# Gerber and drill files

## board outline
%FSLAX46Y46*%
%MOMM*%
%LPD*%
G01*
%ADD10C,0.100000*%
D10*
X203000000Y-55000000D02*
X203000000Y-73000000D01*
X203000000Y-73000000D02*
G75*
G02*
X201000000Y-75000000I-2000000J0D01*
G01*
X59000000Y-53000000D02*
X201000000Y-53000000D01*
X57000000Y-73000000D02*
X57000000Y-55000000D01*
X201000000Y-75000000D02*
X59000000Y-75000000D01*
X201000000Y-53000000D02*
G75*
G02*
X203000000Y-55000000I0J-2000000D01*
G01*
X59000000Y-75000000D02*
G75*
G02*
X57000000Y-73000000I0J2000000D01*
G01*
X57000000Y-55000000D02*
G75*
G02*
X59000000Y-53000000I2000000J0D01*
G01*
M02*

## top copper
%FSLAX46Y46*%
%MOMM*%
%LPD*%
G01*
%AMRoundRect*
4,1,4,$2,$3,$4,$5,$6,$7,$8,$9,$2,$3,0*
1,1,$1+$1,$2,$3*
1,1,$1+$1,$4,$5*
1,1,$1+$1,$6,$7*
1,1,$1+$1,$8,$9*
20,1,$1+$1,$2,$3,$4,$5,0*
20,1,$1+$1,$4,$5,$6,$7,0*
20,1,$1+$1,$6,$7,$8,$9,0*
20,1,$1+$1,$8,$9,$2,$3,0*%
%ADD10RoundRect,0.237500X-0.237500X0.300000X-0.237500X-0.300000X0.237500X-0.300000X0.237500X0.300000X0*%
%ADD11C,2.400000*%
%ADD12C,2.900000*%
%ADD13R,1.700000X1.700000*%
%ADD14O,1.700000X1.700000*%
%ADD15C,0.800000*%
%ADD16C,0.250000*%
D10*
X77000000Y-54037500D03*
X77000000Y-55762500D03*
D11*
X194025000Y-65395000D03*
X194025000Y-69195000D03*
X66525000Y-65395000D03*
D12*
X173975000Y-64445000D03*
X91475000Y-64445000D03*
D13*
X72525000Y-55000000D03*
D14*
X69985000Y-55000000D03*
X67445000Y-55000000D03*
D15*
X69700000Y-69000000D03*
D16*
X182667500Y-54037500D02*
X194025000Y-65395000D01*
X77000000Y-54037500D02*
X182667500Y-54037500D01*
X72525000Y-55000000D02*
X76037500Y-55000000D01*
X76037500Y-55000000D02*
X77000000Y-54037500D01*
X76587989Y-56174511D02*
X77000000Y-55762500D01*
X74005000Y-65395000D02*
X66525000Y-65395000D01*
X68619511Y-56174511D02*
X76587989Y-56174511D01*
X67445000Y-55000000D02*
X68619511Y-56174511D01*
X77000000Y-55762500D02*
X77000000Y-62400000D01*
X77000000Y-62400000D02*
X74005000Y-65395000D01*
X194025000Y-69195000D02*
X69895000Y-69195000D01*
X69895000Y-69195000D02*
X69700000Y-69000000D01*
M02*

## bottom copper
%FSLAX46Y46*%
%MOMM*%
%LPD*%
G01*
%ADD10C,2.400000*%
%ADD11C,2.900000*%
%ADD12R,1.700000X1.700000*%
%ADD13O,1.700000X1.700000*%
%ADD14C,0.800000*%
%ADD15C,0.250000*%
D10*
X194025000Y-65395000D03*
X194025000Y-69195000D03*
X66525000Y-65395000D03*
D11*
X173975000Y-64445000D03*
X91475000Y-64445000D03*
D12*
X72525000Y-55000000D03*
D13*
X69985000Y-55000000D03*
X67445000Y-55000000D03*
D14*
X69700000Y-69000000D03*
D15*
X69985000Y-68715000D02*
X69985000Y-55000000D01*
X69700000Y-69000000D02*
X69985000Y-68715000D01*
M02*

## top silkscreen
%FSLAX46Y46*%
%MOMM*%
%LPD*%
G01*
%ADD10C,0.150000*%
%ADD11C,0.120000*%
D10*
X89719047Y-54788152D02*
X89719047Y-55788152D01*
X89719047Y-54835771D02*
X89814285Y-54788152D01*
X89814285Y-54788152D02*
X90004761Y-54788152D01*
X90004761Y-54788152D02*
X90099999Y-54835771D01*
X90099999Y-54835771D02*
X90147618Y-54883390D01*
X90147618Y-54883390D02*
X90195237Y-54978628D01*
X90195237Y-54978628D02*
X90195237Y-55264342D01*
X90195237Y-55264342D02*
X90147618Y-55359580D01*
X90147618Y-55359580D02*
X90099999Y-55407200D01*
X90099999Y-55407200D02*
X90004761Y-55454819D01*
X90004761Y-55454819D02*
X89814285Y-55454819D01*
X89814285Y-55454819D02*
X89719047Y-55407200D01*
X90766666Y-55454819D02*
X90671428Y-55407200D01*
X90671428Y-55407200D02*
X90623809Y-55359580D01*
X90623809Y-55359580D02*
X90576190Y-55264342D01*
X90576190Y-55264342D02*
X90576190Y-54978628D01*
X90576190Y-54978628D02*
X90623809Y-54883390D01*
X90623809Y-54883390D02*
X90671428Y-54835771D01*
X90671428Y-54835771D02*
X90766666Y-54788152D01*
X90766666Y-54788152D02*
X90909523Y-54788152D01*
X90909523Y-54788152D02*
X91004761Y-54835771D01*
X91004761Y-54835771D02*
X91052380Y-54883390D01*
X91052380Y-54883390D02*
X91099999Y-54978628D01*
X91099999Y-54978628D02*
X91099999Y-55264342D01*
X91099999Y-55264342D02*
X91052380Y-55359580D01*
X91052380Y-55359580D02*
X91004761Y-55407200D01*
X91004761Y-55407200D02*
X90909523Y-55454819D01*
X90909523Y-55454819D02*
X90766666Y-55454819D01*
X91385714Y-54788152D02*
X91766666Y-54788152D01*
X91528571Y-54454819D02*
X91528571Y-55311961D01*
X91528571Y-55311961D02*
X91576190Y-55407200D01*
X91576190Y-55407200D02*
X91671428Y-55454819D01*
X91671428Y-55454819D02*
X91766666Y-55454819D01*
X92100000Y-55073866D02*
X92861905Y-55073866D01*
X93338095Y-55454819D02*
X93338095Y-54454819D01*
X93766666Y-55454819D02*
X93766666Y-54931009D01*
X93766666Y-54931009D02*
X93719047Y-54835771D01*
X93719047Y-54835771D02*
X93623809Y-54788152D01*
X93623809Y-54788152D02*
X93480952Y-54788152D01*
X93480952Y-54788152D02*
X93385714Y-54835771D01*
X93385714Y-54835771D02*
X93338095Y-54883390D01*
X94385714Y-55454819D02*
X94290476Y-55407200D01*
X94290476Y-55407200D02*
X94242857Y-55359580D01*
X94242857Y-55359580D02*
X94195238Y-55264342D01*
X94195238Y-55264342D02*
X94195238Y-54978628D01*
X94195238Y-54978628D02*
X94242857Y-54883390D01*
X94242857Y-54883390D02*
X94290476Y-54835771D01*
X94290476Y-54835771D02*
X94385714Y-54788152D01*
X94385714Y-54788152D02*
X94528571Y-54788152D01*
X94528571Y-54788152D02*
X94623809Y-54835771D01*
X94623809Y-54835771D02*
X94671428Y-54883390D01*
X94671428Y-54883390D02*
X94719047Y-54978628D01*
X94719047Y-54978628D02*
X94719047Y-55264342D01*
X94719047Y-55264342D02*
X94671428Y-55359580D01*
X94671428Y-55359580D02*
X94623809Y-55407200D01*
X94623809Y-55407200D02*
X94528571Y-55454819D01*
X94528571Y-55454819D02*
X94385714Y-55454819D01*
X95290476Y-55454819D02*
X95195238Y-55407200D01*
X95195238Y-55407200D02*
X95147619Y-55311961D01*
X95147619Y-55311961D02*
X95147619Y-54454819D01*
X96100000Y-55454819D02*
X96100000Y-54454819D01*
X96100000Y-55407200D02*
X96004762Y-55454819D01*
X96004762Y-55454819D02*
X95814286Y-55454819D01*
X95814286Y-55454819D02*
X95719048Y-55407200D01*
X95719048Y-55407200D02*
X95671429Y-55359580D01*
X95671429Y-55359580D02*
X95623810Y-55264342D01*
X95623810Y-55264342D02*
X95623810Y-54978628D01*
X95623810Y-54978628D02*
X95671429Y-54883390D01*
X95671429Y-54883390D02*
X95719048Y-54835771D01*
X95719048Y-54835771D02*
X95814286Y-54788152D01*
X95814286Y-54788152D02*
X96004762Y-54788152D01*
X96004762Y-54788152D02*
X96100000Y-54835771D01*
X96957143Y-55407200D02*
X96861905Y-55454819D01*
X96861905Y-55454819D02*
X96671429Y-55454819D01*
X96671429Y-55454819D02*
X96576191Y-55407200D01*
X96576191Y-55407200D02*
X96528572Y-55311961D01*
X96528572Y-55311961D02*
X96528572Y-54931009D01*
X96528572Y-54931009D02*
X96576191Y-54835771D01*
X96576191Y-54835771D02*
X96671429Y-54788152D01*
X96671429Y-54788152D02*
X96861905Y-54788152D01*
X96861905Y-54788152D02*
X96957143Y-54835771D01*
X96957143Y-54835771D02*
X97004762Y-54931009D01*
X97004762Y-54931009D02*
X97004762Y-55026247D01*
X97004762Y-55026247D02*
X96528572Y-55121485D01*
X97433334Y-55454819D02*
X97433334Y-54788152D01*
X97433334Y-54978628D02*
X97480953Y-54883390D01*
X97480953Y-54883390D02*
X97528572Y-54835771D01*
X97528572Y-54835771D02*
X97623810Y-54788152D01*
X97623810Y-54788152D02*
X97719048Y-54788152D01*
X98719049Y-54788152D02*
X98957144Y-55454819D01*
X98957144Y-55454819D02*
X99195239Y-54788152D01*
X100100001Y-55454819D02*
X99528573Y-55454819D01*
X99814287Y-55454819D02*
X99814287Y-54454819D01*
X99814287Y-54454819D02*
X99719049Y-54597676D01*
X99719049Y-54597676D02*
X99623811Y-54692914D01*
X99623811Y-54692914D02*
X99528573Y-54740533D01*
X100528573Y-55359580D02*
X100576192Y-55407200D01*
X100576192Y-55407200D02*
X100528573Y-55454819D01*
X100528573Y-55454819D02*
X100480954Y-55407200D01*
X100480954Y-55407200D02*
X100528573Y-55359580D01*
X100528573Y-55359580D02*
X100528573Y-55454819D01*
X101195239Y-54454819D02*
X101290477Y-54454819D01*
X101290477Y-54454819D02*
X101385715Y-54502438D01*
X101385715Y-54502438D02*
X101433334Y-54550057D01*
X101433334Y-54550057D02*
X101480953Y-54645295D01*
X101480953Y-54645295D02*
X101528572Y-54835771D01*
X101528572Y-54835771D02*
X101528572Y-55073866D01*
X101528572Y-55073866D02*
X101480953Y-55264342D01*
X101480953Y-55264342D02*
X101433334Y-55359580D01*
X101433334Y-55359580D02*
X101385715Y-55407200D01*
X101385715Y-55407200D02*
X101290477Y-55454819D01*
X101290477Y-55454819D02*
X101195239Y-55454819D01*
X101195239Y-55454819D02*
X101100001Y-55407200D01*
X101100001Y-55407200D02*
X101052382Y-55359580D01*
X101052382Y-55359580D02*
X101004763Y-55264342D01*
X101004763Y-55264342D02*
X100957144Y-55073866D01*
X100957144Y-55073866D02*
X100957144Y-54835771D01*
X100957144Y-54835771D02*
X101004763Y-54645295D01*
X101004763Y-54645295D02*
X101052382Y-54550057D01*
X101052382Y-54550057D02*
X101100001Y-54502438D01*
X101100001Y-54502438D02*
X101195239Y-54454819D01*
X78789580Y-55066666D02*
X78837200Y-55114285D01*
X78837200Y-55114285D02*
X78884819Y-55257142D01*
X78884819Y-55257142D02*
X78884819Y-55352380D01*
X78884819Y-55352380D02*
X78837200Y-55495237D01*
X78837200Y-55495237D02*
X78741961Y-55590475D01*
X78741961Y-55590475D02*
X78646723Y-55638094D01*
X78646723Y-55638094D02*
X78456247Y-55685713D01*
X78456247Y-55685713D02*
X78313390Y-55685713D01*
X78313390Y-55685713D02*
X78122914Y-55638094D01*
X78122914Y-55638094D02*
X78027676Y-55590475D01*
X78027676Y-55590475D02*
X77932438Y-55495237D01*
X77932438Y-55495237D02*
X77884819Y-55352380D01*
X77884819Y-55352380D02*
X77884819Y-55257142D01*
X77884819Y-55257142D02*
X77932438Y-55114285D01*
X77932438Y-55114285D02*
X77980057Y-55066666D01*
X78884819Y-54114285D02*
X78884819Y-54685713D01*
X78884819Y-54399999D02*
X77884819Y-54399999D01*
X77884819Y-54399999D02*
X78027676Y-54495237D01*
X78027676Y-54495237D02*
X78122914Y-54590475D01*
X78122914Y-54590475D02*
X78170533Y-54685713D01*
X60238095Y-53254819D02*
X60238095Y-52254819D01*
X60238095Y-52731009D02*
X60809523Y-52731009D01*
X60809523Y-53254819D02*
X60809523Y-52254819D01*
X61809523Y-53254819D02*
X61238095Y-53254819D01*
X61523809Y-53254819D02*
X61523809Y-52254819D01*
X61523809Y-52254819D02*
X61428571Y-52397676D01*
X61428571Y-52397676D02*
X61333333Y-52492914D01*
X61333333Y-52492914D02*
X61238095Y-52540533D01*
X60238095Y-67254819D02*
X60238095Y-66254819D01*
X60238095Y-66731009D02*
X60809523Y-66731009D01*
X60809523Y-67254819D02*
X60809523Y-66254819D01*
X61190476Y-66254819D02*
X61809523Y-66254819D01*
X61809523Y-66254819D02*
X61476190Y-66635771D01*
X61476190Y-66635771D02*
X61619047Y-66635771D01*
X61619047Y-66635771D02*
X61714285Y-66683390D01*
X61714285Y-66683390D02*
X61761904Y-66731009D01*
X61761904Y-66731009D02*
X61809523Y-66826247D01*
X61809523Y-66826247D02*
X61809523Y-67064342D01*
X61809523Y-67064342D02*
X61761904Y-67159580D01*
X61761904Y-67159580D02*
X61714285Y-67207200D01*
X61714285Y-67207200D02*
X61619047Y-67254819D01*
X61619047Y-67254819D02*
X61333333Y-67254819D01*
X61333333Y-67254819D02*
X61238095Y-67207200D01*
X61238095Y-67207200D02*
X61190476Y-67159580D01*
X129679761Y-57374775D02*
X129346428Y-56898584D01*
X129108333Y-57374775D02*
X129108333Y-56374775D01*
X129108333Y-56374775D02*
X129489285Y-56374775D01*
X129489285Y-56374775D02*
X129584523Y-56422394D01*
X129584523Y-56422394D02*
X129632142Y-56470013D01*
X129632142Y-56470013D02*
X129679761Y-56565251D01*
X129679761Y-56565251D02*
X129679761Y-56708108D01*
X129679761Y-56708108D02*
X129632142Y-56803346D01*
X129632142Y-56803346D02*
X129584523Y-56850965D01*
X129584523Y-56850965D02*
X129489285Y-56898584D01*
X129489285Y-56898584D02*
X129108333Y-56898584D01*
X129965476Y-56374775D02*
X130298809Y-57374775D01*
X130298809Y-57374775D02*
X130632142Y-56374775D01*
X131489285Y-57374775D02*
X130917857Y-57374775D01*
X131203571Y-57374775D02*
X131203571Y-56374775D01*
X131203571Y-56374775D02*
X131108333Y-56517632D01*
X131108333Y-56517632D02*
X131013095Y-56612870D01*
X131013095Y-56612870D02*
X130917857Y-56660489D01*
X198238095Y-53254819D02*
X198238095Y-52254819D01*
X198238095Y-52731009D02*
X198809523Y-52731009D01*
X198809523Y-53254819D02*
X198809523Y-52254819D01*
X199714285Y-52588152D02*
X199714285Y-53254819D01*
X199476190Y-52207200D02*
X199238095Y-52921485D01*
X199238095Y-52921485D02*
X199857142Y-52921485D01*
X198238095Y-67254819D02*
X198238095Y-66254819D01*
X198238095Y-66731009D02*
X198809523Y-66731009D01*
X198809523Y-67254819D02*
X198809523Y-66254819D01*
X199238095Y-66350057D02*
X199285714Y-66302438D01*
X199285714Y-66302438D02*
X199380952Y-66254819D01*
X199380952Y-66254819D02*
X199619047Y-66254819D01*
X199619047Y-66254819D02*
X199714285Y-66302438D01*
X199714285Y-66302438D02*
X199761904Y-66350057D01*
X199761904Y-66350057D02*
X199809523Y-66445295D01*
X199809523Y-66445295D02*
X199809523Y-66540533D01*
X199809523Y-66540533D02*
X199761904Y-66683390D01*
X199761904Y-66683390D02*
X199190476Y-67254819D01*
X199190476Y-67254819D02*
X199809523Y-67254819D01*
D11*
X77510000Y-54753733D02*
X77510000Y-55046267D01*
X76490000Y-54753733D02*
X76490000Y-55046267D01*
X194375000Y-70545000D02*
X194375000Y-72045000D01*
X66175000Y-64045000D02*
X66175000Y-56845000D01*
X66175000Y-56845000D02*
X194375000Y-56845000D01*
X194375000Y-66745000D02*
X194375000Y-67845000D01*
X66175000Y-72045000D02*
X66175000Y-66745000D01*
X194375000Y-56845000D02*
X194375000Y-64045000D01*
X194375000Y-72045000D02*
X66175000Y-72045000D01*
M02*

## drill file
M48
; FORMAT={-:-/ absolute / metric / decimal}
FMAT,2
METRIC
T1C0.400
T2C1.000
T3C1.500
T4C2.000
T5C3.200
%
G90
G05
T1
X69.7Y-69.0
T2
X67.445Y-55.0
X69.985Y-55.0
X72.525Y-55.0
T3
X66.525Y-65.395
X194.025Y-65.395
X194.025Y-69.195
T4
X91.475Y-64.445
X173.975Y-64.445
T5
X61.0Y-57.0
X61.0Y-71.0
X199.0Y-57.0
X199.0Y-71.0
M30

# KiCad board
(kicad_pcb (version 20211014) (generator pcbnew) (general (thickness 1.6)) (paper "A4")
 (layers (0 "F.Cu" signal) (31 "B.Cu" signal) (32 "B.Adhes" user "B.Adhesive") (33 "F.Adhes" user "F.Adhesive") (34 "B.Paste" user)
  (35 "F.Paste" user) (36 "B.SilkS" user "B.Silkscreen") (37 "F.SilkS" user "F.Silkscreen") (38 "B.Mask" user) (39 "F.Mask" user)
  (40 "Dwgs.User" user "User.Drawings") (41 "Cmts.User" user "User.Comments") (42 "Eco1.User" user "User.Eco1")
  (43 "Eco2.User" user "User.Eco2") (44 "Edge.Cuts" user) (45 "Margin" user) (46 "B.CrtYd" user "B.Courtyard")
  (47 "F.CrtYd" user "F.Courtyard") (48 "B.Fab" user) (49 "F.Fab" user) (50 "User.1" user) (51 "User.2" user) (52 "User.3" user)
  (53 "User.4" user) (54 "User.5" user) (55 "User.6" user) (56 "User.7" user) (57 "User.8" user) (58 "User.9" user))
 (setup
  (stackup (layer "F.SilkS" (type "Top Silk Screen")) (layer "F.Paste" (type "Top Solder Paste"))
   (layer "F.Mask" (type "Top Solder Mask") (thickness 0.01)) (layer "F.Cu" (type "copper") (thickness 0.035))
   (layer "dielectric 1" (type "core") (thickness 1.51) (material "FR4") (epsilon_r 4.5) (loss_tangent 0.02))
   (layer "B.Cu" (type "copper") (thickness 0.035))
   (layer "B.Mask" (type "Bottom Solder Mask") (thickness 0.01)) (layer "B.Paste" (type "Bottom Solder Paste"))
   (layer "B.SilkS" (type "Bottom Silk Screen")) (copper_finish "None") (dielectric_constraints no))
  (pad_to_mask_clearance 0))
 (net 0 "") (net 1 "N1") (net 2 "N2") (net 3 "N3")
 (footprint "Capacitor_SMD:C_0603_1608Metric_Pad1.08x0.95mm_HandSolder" (layer "F.Cu") (at 77 54.9 -90)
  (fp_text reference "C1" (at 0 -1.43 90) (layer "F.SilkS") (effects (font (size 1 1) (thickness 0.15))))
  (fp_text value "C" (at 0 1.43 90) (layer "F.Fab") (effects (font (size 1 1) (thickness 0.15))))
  (fp_line (start -0.146267 -0.51) (end 0.146267 -0.51) (layer "F.SilkS") (width 0.12))
  (fp_line (start -0.146267 0.51) (end 0.146267 0.51) (layer "F.SilkS") (width 0.12))
  (pad "1" smd roundrect (at -0.8625 0 270) (size 1.075 0.95) (layers "F.Cu" "F.Paste" "F.Mask") (roundrect_rratio 0.25) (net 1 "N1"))
  (pad "2" smd roundrect (at 0.8625 0 270) (size 1.075 0.95) (layers "F.Cu" "F.Paste" "F.Mask") (roundrect_rratio 0.25) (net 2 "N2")))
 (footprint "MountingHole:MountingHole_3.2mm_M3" (layer "F.Cu") (at 61 57)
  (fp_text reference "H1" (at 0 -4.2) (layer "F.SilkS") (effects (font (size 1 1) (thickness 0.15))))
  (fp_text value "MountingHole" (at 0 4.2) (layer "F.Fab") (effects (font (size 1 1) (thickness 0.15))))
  (pad "" np_thru_hole circle (at 0 0) (size 3.2 3.2) (drill 3.2) (layers *.Cu *.Mask)))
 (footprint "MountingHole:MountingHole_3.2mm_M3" (layer "F.Cu") (at 61 71)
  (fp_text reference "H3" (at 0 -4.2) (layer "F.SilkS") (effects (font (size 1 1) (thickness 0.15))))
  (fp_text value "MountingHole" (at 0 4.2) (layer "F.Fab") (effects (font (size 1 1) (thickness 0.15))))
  (pad "" np_thru_hole circle (at 0 0) (size 3.2 3.2) (drill 3.2) (layers *.Cu *.Mask)))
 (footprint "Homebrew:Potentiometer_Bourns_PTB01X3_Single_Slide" (layer "F.Cu") (at 130.275 64.445)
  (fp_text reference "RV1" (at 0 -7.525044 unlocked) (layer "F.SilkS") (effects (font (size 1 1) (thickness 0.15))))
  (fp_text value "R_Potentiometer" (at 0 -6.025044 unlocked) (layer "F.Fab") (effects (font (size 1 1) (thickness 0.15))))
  (fp_line (start 64.1 6.1) (end 64.1 7.6) (layer "F.SilkS") (width 0.12))
  (fp_line (start -64.1 -0.4) (end -64.1 -7.6) (layer "F.SilkS") (width 0.12))
  (fp_line (start -64.1 -7.6) (end 64.1 -7.6) (layer "F.SilkS") (width 0.12))
  (fp_line (start 64.1 2.3) (end 64.1 3.4) (layer "F.SilkS") (width 0.12))
  (fp_line (start -64.1 7.6) (end -64.1 2.3) (layer "F.SilkS") (width 0.12))
  (fp_line (start 64.1 -7.6) (end 64.1 -0.4) (layer "F.SilkS") (width 0.12))
  (fp_line (start 64.1 7.6) (end -64.1 7.6) (layer "F.SilkS") (width 0.12))
  (pad "1" thru_hole circle (at 63.75 0.95) (size 2.4 2.4) (drill 1.5) (layers *.Cu *.Mask) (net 1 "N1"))
  (pad "2" thru_hole circle (at 63.75 4.75) (size 2.4 2.4) (drill 1.5) (layers *.Cu *.Mask) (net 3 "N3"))
  (pad "3" thru_hole circle (at -63.75 0.95) (size 2.4 2.4) (drill 1.5) (layers *.Cu *.Mask) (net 2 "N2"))
  (pad "~" thru_hole circle (at 43.7 0) (size 2.9 2.9) (drill 2) (layers *.Cu *.Mask))
  (pad "~" thru_hole circle (at -38.8 0) (size 2.9 2.9) (drill 2) (layers *.Cu *.Mask)))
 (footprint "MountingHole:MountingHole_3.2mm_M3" (layer "F.Cu") (at 199 57)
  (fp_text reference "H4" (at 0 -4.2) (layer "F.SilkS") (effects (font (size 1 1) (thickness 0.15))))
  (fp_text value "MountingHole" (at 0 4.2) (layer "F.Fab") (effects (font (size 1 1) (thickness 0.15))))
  (pad "" np_thru_hole circle (at 0 0) (size 3.2 3.2) (drill 3.2) (layers *.Cu *.Mask)))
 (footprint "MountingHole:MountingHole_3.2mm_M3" (layer "F.Cu") (at 199 71)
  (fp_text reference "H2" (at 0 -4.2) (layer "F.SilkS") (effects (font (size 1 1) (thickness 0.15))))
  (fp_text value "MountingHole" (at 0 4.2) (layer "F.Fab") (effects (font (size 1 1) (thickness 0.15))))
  (pad "" np_thru_hole circle (at 0 0) (size 3.2 3.2) (drill 3.2) (layers *.Cu *.Mask)))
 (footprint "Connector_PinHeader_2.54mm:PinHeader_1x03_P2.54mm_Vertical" (layer "B.Cu") (at 72.525 55 90)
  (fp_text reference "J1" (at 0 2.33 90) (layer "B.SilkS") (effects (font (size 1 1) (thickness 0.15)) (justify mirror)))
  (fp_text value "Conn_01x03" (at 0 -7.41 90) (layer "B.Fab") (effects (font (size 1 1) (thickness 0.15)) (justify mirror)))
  (pad "1" thru_hole rect (at 0 0 90) (size 1.7 1.7) (drill 1) (layers *.Cu *.Mask) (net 1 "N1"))
  (pad "2" thru_hole oval (at 0 -2.54 90) (size 1.7 1.7) (drill 1) (layers *.Cu *.Mask) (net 3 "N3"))
  (pad "3" thru_hole oval (at 0 -5.08 90) (size 1.7 1.7) (drill 1) (layers *.Cu *.Mask) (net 2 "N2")))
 (gr_line (start 203 55) (end 203 73) (layer "Edge.Cuts") (width 0.1))
 (gr_arc (start 203 73) (mid 202.414214 74.414214) (end 201 75) (layer "Edge.Cuts") (width 0.1))
 (gr_line (start 59 53) (end 201 53) (layer "Edge.Cuts") (width 0.1))
 (gr_line (start 57 73) (end 57 55) (layer "Edge.Cuts") (width 0.1))
 (gr_line (start 201 75) (end 59 75) (layer "Edge.Cuts") (width 0.1))
 (gr_arc (start 201 53) (mid 202.414214 53.585786) (end 203 55) (layer "Edge.Cuts") (width 0.1))
 (gr_arc (start 59 75) (mid 57.585786 74.414214) (end 57 73) (layer "Edge.Cuts") (width 0.1))
 (gr_arc (start 57 55) (mid 57.585786 53.585786) (end 59 53) (layer "Edge.Cuts") (width 0.1))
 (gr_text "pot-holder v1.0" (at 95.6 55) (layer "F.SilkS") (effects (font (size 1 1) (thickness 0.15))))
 (segment (start 182.6675 54.0375) (end 194.025 65.395) (width 0.25) (layer "F.Cu") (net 1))
 (segment (start 77 54.0375) (end 182.6675 54.0375) (width 0.25) (layer "F.Cu") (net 1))
 (segment (start 72.525 55) (end 76.0375 55) (width 0.25) (layer "F.Cu") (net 1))
 (segment (start 76.0375 55) (end 77 54.0375) (width 0.25) (layer "F.Cu") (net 1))
 (segment (start 76.587989 56.174511) (end 77 55.7625) (width 0.25) (layer "F.Cu") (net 2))
 (segment (start 74.005 65.395) (end 66.525 65.395) (width 0.25) (layer "F.Cu") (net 2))
 (segment (start 68.619511 56.174511) (end 76.587989 56.174511) (width 0.25) (layer "F.Cu") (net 2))
 (segment (start 67.445 55) (end 68.619511 56.174511) (width 0.25) (layer "F.Cu") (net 2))
 (segment (start 77 55.7625) (end 77 62.4) (width 0.25) (layer "F.Cu") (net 2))
 (segment (start 77 62.4) (end 74.005 65.395) (width 0.25) (layer "F.Cu") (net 2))
 (segment (start 194.025 69.195) (end 69.895 69.195) (width 0.25) (layer "F.Cu") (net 3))
 (segment (start 69.895 69.195) (end 69.7 69) (width 0.25) (layer "F.Cu") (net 3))
 (via (at 69.7 69) (size 0.8) (drill 0.4) (layers "F.Cu" "B.Cu") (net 3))
 (segment (start 69.985 68.715) (end 69.985 55) (width 0.25) (layer "B.Cu") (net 3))
 (segment (start 69.7 69) (end 69.985 68.715) (width 0.25) (layer "B.Cu") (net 3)))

